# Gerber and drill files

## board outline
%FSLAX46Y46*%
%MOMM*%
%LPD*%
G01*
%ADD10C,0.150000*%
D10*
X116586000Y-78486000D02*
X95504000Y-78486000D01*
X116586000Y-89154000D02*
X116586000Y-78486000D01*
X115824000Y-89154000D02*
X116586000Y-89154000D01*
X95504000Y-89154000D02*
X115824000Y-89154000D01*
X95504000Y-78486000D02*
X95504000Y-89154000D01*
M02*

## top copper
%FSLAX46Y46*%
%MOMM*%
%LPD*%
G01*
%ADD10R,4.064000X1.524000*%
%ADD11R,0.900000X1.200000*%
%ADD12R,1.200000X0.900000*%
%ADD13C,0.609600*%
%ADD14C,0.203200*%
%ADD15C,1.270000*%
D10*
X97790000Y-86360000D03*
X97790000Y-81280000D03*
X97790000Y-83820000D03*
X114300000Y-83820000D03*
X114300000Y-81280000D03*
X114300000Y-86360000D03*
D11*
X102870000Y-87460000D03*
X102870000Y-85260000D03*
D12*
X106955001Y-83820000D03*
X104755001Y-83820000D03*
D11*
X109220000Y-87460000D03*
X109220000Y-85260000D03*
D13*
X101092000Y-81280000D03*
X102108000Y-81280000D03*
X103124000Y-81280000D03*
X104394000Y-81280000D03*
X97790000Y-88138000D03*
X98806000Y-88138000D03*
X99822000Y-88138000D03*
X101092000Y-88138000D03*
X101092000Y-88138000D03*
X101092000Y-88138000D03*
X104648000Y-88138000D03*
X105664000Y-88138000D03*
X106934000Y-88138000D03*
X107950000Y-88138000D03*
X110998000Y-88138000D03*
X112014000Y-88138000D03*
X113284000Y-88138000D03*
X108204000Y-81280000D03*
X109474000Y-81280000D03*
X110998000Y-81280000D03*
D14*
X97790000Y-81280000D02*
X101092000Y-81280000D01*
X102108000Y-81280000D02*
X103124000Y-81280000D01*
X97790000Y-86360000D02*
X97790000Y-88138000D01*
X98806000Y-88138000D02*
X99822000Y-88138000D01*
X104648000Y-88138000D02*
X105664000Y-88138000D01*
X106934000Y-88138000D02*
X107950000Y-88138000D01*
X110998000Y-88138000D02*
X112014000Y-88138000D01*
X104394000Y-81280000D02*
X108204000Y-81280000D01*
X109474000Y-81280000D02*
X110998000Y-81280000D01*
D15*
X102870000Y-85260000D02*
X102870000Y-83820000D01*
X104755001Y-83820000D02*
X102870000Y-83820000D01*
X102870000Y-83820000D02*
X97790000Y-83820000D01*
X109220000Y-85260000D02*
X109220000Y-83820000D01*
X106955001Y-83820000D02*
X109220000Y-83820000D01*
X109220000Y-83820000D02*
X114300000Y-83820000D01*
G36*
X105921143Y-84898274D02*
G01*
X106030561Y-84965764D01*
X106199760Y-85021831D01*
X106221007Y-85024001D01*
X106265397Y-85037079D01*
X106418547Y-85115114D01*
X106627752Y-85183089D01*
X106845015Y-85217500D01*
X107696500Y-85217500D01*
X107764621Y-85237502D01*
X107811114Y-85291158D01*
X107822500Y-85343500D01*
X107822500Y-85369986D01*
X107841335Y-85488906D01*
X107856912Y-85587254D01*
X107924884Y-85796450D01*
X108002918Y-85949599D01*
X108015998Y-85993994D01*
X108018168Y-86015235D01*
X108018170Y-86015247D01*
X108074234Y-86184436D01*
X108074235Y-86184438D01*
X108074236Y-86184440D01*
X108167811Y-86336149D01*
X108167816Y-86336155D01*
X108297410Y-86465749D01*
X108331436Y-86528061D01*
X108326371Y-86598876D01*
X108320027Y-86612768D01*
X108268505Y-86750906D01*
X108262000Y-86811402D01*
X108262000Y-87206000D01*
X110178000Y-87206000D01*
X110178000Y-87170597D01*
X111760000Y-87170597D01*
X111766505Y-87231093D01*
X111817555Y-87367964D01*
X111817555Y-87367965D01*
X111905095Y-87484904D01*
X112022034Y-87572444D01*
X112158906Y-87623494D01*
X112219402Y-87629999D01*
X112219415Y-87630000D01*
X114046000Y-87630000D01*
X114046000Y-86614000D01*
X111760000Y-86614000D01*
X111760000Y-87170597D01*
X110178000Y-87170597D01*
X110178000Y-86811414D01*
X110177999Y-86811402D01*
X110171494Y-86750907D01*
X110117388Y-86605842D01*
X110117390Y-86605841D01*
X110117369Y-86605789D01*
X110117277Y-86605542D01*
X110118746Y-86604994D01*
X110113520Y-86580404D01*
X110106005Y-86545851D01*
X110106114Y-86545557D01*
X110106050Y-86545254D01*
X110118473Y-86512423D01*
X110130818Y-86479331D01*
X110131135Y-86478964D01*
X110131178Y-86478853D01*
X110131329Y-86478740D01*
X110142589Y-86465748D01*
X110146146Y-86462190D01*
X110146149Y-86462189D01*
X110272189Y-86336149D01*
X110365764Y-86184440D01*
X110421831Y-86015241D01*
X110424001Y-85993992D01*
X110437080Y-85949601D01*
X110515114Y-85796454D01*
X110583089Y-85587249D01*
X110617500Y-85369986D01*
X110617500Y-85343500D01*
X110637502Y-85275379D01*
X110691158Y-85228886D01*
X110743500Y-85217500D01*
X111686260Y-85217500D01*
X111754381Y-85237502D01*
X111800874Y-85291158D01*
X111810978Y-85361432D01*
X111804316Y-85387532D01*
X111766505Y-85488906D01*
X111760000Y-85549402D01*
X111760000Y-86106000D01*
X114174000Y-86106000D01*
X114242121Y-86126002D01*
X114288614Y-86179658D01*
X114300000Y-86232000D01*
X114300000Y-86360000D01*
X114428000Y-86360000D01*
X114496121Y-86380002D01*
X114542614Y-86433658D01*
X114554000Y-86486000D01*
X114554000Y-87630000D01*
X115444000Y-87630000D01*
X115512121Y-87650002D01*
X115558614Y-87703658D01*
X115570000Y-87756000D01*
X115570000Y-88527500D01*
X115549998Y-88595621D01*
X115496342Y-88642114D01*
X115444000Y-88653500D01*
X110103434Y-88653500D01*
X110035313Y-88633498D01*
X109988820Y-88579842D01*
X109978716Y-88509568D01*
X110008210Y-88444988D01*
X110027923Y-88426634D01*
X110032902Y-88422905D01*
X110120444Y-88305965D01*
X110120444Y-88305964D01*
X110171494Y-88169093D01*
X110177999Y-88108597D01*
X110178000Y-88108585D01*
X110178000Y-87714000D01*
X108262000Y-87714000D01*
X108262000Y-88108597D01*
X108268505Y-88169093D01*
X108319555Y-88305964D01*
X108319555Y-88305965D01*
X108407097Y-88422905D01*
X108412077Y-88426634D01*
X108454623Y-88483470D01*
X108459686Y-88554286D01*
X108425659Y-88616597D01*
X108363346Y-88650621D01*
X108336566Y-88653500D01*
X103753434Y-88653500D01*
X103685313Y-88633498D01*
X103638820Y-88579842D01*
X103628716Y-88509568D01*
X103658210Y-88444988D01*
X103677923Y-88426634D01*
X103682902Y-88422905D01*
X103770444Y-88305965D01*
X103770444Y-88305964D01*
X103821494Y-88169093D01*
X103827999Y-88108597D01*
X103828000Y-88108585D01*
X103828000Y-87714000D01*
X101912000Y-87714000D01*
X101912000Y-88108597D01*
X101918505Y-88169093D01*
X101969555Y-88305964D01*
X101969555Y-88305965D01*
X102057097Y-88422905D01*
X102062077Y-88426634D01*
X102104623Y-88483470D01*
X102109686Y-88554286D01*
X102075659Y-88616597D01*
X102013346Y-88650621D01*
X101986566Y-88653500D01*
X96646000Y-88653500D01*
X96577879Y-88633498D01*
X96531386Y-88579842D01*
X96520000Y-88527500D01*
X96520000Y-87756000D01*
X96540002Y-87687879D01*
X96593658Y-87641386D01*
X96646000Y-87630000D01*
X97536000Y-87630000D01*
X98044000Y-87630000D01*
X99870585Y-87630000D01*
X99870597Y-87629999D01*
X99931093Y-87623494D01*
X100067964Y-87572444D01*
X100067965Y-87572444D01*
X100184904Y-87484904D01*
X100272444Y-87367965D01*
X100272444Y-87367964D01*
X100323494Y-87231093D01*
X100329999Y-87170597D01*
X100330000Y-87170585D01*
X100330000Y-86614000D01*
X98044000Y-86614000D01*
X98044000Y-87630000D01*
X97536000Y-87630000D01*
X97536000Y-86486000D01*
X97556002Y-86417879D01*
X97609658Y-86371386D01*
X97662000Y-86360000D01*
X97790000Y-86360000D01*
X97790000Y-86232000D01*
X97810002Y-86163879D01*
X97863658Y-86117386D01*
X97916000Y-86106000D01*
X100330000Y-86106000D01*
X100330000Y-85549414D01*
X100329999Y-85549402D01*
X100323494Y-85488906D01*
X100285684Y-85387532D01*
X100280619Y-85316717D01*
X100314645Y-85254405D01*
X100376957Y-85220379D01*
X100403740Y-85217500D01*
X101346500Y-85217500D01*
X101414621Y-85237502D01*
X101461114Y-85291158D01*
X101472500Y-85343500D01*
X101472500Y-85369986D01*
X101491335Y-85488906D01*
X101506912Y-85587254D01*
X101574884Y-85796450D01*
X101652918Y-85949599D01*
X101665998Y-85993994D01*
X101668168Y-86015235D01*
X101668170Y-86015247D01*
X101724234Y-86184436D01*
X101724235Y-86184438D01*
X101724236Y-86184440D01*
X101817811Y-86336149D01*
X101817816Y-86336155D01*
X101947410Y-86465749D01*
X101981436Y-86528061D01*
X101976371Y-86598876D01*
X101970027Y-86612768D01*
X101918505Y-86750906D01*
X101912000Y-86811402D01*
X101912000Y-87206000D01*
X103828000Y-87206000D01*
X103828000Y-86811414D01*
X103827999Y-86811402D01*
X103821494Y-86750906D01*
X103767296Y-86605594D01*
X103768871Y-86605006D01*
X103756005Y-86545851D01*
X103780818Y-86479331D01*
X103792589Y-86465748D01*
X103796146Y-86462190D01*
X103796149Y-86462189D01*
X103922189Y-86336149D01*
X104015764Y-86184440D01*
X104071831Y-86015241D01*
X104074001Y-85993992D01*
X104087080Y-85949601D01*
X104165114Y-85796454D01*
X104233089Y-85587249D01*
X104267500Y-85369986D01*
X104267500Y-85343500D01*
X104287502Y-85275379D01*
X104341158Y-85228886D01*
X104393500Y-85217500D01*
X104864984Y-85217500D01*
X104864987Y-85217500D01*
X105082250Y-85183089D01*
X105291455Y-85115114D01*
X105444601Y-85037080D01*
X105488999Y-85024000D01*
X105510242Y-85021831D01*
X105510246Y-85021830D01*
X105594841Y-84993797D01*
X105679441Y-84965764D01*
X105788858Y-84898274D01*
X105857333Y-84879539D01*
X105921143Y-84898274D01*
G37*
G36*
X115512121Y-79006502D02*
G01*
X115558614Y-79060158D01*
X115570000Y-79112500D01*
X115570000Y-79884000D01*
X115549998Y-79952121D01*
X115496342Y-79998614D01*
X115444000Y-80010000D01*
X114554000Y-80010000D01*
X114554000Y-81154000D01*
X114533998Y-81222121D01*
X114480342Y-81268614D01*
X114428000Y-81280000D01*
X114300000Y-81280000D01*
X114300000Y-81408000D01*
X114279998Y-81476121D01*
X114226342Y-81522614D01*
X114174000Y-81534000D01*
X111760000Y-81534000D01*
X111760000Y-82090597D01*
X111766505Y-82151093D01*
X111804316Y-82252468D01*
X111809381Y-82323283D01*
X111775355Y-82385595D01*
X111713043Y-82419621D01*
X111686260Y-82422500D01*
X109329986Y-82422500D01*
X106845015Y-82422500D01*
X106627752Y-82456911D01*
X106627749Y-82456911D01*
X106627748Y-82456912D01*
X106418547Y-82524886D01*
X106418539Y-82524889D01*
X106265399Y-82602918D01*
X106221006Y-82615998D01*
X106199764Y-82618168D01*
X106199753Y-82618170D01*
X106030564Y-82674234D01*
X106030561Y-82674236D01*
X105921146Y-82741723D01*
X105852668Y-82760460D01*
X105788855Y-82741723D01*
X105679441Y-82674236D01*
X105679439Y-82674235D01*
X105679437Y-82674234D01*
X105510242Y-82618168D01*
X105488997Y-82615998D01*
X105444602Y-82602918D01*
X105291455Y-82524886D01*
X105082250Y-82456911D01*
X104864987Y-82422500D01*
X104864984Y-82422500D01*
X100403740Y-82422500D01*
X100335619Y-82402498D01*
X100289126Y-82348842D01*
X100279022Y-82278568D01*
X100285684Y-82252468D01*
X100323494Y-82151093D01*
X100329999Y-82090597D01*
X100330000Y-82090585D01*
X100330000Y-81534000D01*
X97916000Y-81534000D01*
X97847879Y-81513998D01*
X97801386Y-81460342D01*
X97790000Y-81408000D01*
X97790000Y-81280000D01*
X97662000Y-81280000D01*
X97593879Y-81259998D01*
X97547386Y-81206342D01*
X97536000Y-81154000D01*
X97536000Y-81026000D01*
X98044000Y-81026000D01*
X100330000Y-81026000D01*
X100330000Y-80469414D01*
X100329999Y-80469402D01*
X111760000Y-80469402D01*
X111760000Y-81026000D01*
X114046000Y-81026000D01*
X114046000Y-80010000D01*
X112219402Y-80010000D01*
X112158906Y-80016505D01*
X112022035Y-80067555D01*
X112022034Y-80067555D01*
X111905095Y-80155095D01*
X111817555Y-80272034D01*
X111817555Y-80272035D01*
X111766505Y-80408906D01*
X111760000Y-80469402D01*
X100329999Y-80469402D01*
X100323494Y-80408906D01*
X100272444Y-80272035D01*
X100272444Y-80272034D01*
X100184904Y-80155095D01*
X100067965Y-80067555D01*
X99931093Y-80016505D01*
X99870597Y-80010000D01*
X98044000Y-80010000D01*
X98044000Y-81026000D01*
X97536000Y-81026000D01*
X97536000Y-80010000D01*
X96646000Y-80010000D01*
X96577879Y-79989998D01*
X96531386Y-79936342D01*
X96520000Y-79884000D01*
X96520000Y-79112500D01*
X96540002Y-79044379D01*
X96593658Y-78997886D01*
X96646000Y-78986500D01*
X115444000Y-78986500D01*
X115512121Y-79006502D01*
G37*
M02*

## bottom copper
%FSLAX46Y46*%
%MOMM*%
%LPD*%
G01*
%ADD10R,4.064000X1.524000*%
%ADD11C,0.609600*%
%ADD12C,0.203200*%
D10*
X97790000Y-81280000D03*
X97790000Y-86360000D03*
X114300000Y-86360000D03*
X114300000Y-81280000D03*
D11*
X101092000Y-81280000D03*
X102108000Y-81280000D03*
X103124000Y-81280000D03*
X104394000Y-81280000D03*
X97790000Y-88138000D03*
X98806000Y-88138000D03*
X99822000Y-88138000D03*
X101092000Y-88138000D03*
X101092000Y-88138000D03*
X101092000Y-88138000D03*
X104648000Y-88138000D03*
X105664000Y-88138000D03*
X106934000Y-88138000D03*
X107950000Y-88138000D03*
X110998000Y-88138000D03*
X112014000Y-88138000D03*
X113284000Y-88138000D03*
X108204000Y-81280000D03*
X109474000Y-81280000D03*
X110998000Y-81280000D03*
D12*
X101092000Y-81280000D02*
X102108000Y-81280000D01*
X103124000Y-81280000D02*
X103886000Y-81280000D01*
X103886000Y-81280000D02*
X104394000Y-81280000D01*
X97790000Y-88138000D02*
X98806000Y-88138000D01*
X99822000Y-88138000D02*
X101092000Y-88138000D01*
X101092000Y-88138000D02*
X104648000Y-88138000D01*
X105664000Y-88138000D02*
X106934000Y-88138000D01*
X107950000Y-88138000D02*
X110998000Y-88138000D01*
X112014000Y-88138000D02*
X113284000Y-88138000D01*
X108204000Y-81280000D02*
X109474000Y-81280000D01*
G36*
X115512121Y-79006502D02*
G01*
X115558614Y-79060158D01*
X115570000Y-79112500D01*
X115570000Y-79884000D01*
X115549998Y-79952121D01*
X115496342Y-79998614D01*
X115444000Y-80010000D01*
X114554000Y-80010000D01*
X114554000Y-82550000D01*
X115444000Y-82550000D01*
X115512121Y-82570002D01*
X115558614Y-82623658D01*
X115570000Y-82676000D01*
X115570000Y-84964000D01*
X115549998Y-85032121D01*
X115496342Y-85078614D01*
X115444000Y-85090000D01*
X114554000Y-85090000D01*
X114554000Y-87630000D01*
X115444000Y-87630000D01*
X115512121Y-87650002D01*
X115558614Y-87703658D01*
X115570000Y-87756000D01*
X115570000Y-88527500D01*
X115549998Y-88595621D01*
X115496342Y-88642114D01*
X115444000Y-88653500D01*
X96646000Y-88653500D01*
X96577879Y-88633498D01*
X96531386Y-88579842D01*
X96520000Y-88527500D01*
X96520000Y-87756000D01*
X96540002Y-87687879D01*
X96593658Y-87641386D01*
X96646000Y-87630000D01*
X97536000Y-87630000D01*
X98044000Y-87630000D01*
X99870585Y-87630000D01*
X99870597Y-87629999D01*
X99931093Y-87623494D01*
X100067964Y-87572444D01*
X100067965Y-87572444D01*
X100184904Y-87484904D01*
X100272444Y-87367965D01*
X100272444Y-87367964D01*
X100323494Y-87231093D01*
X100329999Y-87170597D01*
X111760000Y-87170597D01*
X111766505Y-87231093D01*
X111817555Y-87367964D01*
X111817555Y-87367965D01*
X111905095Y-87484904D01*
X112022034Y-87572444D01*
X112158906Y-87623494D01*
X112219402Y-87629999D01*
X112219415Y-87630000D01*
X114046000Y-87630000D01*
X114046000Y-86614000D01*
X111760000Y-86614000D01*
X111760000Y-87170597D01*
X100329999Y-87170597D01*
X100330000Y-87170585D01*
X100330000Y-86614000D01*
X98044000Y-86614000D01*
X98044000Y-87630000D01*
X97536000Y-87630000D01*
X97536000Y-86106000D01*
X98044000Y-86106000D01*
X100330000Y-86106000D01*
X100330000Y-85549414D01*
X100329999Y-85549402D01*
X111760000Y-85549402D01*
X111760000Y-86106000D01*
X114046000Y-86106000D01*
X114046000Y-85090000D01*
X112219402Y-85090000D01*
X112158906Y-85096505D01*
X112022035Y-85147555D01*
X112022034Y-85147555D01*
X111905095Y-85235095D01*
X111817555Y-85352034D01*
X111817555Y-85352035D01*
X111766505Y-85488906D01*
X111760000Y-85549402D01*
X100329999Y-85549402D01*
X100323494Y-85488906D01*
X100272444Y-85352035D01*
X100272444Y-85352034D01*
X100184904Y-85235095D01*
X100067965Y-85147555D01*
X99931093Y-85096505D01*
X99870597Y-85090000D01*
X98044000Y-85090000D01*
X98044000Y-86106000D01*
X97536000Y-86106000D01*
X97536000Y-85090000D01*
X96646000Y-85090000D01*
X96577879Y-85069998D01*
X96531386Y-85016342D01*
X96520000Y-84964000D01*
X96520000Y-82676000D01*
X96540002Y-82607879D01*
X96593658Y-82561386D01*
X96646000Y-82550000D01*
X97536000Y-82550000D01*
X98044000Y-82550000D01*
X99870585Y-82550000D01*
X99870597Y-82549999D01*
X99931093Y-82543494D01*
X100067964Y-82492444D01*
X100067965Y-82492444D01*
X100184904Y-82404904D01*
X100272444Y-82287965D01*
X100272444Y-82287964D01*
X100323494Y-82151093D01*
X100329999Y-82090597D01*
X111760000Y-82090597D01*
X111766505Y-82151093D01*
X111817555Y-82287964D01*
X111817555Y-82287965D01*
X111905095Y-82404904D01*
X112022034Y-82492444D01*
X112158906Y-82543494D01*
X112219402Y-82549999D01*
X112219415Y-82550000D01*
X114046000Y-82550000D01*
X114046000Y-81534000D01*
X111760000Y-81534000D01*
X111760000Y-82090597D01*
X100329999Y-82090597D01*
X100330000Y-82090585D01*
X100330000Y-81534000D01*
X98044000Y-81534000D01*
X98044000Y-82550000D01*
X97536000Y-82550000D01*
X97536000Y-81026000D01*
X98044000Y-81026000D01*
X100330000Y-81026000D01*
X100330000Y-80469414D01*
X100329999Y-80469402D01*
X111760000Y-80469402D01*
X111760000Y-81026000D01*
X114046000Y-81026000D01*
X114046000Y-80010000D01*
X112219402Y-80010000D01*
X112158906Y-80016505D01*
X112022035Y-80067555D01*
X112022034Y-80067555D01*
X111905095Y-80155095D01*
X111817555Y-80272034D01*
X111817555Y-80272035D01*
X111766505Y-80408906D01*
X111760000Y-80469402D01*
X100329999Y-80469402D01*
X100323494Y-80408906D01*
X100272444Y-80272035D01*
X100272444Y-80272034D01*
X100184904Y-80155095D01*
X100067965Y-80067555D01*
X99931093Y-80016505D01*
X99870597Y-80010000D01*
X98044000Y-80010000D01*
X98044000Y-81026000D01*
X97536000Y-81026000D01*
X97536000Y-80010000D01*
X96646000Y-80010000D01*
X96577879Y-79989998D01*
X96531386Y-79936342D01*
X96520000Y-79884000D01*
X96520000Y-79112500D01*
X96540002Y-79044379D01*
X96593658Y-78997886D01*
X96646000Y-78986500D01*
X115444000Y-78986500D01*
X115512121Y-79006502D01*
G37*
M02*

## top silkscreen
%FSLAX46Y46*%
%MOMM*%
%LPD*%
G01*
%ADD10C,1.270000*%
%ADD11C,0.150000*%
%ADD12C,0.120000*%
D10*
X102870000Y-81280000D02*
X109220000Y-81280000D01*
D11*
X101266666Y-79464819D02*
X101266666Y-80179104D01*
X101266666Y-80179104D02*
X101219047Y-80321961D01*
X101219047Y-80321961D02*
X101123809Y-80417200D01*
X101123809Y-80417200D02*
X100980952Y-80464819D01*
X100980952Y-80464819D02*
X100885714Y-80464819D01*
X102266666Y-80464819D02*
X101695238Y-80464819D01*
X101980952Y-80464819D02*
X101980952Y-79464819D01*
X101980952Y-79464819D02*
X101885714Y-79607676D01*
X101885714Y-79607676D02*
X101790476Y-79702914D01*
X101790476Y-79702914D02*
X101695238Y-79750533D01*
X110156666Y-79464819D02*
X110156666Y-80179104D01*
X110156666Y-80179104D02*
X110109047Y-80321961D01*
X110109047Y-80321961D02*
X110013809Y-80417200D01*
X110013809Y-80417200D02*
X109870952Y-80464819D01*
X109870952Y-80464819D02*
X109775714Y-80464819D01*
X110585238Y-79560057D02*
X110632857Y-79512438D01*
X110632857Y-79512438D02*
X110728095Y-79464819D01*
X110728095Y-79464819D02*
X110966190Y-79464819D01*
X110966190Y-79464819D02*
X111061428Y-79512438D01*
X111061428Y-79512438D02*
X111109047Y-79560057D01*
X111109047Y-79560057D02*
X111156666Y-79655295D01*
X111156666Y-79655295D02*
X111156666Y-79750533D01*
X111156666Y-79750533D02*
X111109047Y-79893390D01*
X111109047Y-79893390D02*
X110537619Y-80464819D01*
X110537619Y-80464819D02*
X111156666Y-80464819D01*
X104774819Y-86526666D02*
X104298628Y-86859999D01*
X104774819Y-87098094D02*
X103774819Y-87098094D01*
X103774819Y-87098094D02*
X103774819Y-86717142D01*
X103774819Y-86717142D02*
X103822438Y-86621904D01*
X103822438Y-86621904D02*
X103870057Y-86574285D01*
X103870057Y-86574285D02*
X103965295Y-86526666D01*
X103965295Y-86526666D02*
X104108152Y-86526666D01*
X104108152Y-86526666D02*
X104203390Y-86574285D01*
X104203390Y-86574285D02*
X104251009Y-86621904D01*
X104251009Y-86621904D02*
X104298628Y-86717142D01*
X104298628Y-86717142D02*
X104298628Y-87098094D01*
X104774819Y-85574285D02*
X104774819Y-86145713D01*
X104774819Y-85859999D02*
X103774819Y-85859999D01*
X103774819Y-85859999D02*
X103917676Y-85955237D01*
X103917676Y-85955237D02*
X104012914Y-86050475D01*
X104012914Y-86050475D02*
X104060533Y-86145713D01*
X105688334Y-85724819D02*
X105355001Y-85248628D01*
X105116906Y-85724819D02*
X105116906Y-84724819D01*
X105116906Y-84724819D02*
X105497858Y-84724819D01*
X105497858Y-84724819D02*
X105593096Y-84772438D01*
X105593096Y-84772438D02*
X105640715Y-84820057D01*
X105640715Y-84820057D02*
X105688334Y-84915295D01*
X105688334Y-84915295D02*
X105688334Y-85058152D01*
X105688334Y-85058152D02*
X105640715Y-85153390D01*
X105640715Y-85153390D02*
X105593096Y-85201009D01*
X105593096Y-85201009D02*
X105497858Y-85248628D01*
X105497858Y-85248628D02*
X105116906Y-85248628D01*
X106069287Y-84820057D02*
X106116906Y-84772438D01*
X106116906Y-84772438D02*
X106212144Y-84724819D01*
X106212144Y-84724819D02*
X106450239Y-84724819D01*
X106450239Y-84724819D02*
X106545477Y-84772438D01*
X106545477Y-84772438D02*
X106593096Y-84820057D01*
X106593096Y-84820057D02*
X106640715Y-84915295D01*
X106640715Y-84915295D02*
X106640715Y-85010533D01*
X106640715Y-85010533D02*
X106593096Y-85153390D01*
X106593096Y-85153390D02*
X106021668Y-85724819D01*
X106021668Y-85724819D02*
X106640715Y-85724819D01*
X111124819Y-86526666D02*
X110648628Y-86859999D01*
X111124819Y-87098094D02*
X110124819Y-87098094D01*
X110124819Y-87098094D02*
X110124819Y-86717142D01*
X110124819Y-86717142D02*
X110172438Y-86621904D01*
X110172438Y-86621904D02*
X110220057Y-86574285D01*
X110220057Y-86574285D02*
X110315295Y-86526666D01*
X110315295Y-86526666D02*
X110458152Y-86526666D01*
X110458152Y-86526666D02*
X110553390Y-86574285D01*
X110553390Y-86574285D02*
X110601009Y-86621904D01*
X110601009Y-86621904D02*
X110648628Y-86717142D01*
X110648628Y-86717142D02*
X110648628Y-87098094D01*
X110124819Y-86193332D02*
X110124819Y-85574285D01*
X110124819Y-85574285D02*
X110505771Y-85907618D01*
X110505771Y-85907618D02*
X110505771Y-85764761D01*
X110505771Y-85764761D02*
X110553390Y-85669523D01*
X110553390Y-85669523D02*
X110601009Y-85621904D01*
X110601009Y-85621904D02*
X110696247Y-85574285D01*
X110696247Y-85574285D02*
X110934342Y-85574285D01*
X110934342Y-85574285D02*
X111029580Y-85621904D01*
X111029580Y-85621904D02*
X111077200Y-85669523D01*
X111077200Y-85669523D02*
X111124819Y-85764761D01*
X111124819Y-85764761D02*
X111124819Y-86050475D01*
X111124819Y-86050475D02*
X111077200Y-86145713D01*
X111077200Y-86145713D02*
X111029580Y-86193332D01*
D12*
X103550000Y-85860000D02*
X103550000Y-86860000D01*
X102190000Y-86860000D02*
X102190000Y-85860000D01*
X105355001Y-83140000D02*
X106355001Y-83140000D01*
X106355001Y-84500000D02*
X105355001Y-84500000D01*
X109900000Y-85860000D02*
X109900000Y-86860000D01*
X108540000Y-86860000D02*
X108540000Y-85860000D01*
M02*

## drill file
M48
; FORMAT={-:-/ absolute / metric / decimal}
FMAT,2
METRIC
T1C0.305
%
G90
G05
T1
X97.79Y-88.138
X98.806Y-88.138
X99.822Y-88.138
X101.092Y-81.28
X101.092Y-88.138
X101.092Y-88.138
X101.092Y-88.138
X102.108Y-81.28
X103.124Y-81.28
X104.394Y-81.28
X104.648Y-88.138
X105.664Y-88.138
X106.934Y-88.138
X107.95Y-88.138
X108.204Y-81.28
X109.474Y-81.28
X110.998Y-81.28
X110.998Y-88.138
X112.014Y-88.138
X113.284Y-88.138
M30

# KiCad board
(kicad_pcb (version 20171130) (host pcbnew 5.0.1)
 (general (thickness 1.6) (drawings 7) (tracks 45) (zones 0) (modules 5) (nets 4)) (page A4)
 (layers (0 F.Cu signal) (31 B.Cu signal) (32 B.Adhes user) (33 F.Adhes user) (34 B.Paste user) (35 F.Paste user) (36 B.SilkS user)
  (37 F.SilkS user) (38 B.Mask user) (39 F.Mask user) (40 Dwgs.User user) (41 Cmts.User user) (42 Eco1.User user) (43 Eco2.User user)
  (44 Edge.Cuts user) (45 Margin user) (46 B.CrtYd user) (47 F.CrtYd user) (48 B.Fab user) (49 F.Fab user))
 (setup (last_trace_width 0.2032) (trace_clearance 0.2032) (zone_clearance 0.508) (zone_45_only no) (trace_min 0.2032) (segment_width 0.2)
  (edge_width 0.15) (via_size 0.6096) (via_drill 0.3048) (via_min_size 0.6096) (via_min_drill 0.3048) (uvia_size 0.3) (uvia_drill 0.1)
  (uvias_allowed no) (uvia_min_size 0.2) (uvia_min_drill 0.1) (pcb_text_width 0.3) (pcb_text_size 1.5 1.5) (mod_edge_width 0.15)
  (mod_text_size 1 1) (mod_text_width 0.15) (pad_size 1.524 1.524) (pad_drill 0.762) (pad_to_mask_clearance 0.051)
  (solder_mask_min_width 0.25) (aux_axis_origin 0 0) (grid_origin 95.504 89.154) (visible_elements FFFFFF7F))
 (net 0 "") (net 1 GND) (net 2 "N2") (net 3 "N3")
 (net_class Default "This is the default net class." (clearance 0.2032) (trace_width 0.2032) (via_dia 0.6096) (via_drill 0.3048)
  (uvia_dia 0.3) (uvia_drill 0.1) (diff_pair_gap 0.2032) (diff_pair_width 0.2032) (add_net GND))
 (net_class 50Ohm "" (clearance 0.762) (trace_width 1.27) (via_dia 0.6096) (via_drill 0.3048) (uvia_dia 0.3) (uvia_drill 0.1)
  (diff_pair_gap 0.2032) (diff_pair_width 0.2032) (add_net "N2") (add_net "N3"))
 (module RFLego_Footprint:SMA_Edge (layer F.Cu) (at 95.758 83.82)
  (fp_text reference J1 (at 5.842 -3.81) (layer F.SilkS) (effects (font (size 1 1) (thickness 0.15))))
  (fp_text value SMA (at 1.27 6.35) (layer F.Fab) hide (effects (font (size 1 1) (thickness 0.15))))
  (pad 2 smd rect (at 2.032 2.54) (size 4.064 1.524) (layers F.Cu F.Mask) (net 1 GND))
  (pad 2 smd rect (at 2.032 -2.54) (size 4.064 1.524) (layers B.Cu B.Mask) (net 1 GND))
  (pad 2 smd rect (at 2.032 2.54) (size 4.064 1.524) (layers B.Cu B.Mask) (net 1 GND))
  (pad 2 smd rect (at 2.032 -2.54) (size 4.064 1.524) (layers F.Cu F.Mask) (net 1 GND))
  (pad 1 smd rect (at 2.032 0) (size 4.064 1.524) (layers F.Cu F.Mask) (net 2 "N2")))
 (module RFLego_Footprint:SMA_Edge (layer F.Cu) (at 112.268 83.82)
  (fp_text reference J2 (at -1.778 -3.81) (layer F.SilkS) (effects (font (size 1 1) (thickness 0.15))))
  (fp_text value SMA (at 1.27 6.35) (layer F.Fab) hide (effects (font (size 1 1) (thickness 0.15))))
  (pad 1 smd rect (at 2.032 0) (size 4.064 1.524) (layers F.Cu F.Mask) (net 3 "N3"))
  (pad 2 smd rect (at 2.032 -2.54) (size 4.064 1.524) (layers F.Cu F.Mask) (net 1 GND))
  (pad 2 smd rect (at 2.032 2.54) (size 4.064 1.524) (layers B.Cu B.Mask) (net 1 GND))
  (pad 2 smd rect (at 2.032 -2.54) (size 4.064 1.524) (layers B.Cu B.Mask) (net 1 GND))
  (pad 2 smd rect (at 2.032 2.54) (size 4.064 1.524) (layers F.Cu F.Mask) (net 1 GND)))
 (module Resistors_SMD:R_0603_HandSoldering (layer F.Cu) (at 102.87 86.36 270)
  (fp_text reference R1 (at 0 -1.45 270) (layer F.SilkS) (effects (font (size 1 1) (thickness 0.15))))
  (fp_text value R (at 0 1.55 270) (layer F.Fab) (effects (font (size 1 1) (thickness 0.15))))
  (fp_line (start -0.5 -0.68) (end 0.5 -0.68) (layer F.SilkS) (width 0.12))
  (fp_line (start 0.5 0.68) (end -0.5 0.68) (layer F.SilkS) (width 0.12))
  (pad 2 smd rect (at 1.1 0 270) (size 1.2 0.9) (layers F.Cu F.Paste F.Mask) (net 1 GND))
  (pad 1 smd rect (at -1.1 0 270) (size 1.2 0.9) (layers F.Cu F.Paste F.Mask) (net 2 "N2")))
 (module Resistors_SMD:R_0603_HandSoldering (layer F.Cu) (at 105.855001 83.82 180)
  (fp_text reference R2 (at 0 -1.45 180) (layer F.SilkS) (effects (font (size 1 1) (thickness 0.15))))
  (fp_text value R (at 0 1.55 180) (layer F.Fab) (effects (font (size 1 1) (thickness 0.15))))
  (fp_line (start 0.5 0.68) (end -0.5 0.68) (layer F.SilkS) (width 0.12))
  (fp_line (start -0.5 -0.68) (end 0.5 -0.68) (layer F.SilkS) (width 0.12))
  (pad 1 smd rect (at -1.1 0 180) (size 1.2 0.9) (layers F.Cu F.Paste F.Mask) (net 3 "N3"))
  (pad 2 smd rect (at 1.1 0 180) (size 1.2 0.9) (layers F.Cu F.Paste F.Mask) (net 2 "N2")))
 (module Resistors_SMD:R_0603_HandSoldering (layer F.Cu) (at 109.22 86.36 270)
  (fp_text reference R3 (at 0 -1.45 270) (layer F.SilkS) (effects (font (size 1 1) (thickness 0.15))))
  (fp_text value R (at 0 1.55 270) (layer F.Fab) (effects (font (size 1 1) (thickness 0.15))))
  (fp_line (start -0.5 -0.68) (end 0.5 -0.68) (layer F.SilkS) (width 0.12))
  (fp_line (start 0.5 0.68) (end -0.5 0.68) (layer F.SilkS) (width 0.12))
  (pad 2 smd rect (at 1.1 0 270) (size 1.2 0.9) (layers F.Cu F.Paste F.Mask) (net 1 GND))
  (pad 1 smd rect (at -1.1 0 270) (size 1.2 0.9) (layers F.Cu F.Paste F.Mask) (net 3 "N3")))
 (gr_line (start 116.586 78.486) (end 95.504 78.486) (layer Edge.Cuts) (width 0.15))
 (gr_line (start 116.586 89.154) (end 116.586 78.486) (layer Edge.Cuts) (width 0.15))
 (gr_line (start 115.824 89.154) (end 116.586 89.154) (layer Edge.Cuts) (width 0.15))
 (gr_line (start 95.504 89.154) (end 115.824 89.154) (layer Edge.Cuts) (width 0.15))
 (gr_line (start 95.504 78.486) (end 95.504 89.154) (layer Edge.Cuts) (width 0.15))
 (gr_line (start 102.87 81.28) (end 109.22 81.28) (layer F.SilkS) (width 1.27))
 (via (at 101.092 81.28) (size 0.6096) (drill 0.3048) (layers F.Cu B.Cu) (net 1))
 (segment (start 97.79 81.28) (end 101.092 81.28) (width 0.2032) (layer F.Cu) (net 1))
 (via (at 102.108 81.28) (size 0.6096) (drill 0.3048) (layers F.Cu B.Cu) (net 1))
 (segment (start 101.092 81.28) (end 102.108 81.28) (width 0.2032) (layer B.Cu) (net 1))
 (segment (start 102.108 81.28) (end 103.124 81.28) (width 0.2032) (layer F.Cu) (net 1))
 (via (at 103.124 81.28) (size 0.6096) (drill 0.3048) (layers F.Cu B.Cu) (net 1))
 (segment (start 103.124 81.28) (end 103.886 81.28) (width 0.2032) (layer B.Cu) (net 1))
 (via (at 104.394 81.28) (size 0.6096) (drill 0.3048) (layers F.Cu B.Cu) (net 1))
 (segment (start 103.886 81.28) (end 104.394 81.28) (width 0.2032) (layer B.Cu) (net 1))
 (segment (start 97.79 86.36) (end 97.79 88.138) (width 0.2032) (layer F.Cu) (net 1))
 (via (at 97.79 88.138) (size 0.6096) (drill 0.3048) (layers F.Cu B.Cu) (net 1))
 (via (at 98.806 88.138) (size 0.6096) (drill 0.3048) (layers F.Cu B.Cu) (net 1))
 (segment (start 97.79 88.138) (end 98.806 88.138) (width 0.2032) (layer B.Cu) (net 1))
 (via (at 99.822 88.138) (size 0.6096) (drill 0.3048) (layers F.Cu B.Cu) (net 1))
 (segment (start 98.806 88.138) (end 99.822 88.138) (width 0.2032) (layer F.Cu) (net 1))
 (via (at 101.092 88.138) (size 0.6096) (drill 0.3048) (layers F.Cu B.Cu) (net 1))
 (segment (start 99.822 88.138) (end 101.092 88.138) (width 0.2032) (layer B.Cu) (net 1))
 (via (at 101.092 88.138) (size 0.6096) (drill 0.3048) (layers F.Cu B.Cu) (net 1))
 (via (at 101.092 88.138) (size 0.6096) (drill 0.3048) (layers F.Cu B.Cu) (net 1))
 (via (at 104.648 88.138) (size 0.6096) (drill 0.3048) (layers F.Cu B.Cu) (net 1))
 (segment (start 101.092 88.138) (end 104.648 88.138) (width 0.2032) (layer B.Cu) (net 1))
 (via (at 105.664 88.138) (size 0.6096) (drill 0.3048) (layers F.Cu B.Cu) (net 1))
 (segment (start 104.648 88.138) (end 105.664 88.138) (width 0.2032) (layer F.Cu) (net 1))
 (via (at 106.934 88.138) (size 0.6096) (drill 0.3048) (layers F.Cu B.Cu) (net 1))
 (segment (start 105.664 88.138) (end 106.934 88.138) (width 0.2032) (layer B.Cu) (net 1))
 (via (at 107.95 88.138) (size 0.6096) (drill 0.3048) (layers F.Cu B.Cu) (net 1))
 (segment (start 106.934 88.138) (end 107.95 88.138) (width 0.2032) (layer F.Cu) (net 1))
 (via (at 110.998 88.138) (size 0.6096) (drill 0.3048) (layers F.Cu B.Cu) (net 1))
 (segment (start 107.95 88.138) (end 110.998 88.138) (width 0.2032) (layer B.Cu) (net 1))
 (via (at 112.014 88.138) (size 0.6096) (drill 0.3048) (layers F.Cu B.Cu) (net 1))
 (segment (start 110.998 88.138) (end 112.014 88.138) (width 0.2032) (layer F.Cu) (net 1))
 (via (at 113.284 88.138) (size 0.6096) (drill 0.3048) (layers F.Cu B.Cu) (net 1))
 (segment (start 112.014 88.138) (end 113.284 88.138) (width 0.2032) (layer B.Cu) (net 1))
 (via (at 108.204 81.28) (size 0.6096) (drill 0.3048) (layers F.Cu B.Cu) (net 1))
 (segment (start 104.394 81.28) (end 108.204 81.28) (width 0.2032) (layer F.Cu) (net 1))
 (via (at 109.474 81.28) (size 0.6096) (drill 0.3048) (layers F.Cu B.Cu) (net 1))
 (segment (start 108.204 81.28) (end 109.474 81.28) (width 0.2032) (layer B.Cu) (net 1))
 (via (at 110.998 81.28) (size 0.6096) (drill 0.3048) (layers F.Cu B.Cu) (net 1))
 (segment (start 109.474 81.28) (end 110.998 81.28) (width 0.2032) (layer F.Cu) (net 1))
 (segment (start 102.87 85.26) (end 102.87 83.82) (width 1.27) (layer F.Cu) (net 2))
 (segment (start 104.755001 83.82) (end 102.87 83.82) (width 1.27) (layer F.Cu) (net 2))
 (segment (start 102.87 83.82) (end 97.79 83.82) (width 1.27) (layer F.Cu) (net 2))
 (segment (start 109.22 85.26) (end 109.22 83.82) (width 1.27) (layer F.Cu) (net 3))
 (segment (start 106.955001 83.82) (end 109.22 83.82) (width 1.27) (layer F.Cu) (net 3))
 (segment (start 109.22 83.82) (end 114.3 83.82) (width 1.27) (layer F.Cu) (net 3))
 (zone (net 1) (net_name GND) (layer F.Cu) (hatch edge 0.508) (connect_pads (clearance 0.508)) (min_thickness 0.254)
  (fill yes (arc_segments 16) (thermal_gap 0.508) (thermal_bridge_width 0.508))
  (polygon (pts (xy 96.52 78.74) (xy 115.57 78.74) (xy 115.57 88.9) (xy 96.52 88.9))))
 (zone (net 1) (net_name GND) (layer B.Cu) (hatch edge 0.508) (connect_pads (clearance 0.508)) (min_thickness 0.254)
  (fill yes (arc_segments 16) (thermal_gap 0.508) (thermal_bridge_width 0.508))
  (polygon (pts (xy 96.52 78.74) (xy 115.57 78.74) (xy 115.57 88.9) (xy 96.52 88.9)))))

